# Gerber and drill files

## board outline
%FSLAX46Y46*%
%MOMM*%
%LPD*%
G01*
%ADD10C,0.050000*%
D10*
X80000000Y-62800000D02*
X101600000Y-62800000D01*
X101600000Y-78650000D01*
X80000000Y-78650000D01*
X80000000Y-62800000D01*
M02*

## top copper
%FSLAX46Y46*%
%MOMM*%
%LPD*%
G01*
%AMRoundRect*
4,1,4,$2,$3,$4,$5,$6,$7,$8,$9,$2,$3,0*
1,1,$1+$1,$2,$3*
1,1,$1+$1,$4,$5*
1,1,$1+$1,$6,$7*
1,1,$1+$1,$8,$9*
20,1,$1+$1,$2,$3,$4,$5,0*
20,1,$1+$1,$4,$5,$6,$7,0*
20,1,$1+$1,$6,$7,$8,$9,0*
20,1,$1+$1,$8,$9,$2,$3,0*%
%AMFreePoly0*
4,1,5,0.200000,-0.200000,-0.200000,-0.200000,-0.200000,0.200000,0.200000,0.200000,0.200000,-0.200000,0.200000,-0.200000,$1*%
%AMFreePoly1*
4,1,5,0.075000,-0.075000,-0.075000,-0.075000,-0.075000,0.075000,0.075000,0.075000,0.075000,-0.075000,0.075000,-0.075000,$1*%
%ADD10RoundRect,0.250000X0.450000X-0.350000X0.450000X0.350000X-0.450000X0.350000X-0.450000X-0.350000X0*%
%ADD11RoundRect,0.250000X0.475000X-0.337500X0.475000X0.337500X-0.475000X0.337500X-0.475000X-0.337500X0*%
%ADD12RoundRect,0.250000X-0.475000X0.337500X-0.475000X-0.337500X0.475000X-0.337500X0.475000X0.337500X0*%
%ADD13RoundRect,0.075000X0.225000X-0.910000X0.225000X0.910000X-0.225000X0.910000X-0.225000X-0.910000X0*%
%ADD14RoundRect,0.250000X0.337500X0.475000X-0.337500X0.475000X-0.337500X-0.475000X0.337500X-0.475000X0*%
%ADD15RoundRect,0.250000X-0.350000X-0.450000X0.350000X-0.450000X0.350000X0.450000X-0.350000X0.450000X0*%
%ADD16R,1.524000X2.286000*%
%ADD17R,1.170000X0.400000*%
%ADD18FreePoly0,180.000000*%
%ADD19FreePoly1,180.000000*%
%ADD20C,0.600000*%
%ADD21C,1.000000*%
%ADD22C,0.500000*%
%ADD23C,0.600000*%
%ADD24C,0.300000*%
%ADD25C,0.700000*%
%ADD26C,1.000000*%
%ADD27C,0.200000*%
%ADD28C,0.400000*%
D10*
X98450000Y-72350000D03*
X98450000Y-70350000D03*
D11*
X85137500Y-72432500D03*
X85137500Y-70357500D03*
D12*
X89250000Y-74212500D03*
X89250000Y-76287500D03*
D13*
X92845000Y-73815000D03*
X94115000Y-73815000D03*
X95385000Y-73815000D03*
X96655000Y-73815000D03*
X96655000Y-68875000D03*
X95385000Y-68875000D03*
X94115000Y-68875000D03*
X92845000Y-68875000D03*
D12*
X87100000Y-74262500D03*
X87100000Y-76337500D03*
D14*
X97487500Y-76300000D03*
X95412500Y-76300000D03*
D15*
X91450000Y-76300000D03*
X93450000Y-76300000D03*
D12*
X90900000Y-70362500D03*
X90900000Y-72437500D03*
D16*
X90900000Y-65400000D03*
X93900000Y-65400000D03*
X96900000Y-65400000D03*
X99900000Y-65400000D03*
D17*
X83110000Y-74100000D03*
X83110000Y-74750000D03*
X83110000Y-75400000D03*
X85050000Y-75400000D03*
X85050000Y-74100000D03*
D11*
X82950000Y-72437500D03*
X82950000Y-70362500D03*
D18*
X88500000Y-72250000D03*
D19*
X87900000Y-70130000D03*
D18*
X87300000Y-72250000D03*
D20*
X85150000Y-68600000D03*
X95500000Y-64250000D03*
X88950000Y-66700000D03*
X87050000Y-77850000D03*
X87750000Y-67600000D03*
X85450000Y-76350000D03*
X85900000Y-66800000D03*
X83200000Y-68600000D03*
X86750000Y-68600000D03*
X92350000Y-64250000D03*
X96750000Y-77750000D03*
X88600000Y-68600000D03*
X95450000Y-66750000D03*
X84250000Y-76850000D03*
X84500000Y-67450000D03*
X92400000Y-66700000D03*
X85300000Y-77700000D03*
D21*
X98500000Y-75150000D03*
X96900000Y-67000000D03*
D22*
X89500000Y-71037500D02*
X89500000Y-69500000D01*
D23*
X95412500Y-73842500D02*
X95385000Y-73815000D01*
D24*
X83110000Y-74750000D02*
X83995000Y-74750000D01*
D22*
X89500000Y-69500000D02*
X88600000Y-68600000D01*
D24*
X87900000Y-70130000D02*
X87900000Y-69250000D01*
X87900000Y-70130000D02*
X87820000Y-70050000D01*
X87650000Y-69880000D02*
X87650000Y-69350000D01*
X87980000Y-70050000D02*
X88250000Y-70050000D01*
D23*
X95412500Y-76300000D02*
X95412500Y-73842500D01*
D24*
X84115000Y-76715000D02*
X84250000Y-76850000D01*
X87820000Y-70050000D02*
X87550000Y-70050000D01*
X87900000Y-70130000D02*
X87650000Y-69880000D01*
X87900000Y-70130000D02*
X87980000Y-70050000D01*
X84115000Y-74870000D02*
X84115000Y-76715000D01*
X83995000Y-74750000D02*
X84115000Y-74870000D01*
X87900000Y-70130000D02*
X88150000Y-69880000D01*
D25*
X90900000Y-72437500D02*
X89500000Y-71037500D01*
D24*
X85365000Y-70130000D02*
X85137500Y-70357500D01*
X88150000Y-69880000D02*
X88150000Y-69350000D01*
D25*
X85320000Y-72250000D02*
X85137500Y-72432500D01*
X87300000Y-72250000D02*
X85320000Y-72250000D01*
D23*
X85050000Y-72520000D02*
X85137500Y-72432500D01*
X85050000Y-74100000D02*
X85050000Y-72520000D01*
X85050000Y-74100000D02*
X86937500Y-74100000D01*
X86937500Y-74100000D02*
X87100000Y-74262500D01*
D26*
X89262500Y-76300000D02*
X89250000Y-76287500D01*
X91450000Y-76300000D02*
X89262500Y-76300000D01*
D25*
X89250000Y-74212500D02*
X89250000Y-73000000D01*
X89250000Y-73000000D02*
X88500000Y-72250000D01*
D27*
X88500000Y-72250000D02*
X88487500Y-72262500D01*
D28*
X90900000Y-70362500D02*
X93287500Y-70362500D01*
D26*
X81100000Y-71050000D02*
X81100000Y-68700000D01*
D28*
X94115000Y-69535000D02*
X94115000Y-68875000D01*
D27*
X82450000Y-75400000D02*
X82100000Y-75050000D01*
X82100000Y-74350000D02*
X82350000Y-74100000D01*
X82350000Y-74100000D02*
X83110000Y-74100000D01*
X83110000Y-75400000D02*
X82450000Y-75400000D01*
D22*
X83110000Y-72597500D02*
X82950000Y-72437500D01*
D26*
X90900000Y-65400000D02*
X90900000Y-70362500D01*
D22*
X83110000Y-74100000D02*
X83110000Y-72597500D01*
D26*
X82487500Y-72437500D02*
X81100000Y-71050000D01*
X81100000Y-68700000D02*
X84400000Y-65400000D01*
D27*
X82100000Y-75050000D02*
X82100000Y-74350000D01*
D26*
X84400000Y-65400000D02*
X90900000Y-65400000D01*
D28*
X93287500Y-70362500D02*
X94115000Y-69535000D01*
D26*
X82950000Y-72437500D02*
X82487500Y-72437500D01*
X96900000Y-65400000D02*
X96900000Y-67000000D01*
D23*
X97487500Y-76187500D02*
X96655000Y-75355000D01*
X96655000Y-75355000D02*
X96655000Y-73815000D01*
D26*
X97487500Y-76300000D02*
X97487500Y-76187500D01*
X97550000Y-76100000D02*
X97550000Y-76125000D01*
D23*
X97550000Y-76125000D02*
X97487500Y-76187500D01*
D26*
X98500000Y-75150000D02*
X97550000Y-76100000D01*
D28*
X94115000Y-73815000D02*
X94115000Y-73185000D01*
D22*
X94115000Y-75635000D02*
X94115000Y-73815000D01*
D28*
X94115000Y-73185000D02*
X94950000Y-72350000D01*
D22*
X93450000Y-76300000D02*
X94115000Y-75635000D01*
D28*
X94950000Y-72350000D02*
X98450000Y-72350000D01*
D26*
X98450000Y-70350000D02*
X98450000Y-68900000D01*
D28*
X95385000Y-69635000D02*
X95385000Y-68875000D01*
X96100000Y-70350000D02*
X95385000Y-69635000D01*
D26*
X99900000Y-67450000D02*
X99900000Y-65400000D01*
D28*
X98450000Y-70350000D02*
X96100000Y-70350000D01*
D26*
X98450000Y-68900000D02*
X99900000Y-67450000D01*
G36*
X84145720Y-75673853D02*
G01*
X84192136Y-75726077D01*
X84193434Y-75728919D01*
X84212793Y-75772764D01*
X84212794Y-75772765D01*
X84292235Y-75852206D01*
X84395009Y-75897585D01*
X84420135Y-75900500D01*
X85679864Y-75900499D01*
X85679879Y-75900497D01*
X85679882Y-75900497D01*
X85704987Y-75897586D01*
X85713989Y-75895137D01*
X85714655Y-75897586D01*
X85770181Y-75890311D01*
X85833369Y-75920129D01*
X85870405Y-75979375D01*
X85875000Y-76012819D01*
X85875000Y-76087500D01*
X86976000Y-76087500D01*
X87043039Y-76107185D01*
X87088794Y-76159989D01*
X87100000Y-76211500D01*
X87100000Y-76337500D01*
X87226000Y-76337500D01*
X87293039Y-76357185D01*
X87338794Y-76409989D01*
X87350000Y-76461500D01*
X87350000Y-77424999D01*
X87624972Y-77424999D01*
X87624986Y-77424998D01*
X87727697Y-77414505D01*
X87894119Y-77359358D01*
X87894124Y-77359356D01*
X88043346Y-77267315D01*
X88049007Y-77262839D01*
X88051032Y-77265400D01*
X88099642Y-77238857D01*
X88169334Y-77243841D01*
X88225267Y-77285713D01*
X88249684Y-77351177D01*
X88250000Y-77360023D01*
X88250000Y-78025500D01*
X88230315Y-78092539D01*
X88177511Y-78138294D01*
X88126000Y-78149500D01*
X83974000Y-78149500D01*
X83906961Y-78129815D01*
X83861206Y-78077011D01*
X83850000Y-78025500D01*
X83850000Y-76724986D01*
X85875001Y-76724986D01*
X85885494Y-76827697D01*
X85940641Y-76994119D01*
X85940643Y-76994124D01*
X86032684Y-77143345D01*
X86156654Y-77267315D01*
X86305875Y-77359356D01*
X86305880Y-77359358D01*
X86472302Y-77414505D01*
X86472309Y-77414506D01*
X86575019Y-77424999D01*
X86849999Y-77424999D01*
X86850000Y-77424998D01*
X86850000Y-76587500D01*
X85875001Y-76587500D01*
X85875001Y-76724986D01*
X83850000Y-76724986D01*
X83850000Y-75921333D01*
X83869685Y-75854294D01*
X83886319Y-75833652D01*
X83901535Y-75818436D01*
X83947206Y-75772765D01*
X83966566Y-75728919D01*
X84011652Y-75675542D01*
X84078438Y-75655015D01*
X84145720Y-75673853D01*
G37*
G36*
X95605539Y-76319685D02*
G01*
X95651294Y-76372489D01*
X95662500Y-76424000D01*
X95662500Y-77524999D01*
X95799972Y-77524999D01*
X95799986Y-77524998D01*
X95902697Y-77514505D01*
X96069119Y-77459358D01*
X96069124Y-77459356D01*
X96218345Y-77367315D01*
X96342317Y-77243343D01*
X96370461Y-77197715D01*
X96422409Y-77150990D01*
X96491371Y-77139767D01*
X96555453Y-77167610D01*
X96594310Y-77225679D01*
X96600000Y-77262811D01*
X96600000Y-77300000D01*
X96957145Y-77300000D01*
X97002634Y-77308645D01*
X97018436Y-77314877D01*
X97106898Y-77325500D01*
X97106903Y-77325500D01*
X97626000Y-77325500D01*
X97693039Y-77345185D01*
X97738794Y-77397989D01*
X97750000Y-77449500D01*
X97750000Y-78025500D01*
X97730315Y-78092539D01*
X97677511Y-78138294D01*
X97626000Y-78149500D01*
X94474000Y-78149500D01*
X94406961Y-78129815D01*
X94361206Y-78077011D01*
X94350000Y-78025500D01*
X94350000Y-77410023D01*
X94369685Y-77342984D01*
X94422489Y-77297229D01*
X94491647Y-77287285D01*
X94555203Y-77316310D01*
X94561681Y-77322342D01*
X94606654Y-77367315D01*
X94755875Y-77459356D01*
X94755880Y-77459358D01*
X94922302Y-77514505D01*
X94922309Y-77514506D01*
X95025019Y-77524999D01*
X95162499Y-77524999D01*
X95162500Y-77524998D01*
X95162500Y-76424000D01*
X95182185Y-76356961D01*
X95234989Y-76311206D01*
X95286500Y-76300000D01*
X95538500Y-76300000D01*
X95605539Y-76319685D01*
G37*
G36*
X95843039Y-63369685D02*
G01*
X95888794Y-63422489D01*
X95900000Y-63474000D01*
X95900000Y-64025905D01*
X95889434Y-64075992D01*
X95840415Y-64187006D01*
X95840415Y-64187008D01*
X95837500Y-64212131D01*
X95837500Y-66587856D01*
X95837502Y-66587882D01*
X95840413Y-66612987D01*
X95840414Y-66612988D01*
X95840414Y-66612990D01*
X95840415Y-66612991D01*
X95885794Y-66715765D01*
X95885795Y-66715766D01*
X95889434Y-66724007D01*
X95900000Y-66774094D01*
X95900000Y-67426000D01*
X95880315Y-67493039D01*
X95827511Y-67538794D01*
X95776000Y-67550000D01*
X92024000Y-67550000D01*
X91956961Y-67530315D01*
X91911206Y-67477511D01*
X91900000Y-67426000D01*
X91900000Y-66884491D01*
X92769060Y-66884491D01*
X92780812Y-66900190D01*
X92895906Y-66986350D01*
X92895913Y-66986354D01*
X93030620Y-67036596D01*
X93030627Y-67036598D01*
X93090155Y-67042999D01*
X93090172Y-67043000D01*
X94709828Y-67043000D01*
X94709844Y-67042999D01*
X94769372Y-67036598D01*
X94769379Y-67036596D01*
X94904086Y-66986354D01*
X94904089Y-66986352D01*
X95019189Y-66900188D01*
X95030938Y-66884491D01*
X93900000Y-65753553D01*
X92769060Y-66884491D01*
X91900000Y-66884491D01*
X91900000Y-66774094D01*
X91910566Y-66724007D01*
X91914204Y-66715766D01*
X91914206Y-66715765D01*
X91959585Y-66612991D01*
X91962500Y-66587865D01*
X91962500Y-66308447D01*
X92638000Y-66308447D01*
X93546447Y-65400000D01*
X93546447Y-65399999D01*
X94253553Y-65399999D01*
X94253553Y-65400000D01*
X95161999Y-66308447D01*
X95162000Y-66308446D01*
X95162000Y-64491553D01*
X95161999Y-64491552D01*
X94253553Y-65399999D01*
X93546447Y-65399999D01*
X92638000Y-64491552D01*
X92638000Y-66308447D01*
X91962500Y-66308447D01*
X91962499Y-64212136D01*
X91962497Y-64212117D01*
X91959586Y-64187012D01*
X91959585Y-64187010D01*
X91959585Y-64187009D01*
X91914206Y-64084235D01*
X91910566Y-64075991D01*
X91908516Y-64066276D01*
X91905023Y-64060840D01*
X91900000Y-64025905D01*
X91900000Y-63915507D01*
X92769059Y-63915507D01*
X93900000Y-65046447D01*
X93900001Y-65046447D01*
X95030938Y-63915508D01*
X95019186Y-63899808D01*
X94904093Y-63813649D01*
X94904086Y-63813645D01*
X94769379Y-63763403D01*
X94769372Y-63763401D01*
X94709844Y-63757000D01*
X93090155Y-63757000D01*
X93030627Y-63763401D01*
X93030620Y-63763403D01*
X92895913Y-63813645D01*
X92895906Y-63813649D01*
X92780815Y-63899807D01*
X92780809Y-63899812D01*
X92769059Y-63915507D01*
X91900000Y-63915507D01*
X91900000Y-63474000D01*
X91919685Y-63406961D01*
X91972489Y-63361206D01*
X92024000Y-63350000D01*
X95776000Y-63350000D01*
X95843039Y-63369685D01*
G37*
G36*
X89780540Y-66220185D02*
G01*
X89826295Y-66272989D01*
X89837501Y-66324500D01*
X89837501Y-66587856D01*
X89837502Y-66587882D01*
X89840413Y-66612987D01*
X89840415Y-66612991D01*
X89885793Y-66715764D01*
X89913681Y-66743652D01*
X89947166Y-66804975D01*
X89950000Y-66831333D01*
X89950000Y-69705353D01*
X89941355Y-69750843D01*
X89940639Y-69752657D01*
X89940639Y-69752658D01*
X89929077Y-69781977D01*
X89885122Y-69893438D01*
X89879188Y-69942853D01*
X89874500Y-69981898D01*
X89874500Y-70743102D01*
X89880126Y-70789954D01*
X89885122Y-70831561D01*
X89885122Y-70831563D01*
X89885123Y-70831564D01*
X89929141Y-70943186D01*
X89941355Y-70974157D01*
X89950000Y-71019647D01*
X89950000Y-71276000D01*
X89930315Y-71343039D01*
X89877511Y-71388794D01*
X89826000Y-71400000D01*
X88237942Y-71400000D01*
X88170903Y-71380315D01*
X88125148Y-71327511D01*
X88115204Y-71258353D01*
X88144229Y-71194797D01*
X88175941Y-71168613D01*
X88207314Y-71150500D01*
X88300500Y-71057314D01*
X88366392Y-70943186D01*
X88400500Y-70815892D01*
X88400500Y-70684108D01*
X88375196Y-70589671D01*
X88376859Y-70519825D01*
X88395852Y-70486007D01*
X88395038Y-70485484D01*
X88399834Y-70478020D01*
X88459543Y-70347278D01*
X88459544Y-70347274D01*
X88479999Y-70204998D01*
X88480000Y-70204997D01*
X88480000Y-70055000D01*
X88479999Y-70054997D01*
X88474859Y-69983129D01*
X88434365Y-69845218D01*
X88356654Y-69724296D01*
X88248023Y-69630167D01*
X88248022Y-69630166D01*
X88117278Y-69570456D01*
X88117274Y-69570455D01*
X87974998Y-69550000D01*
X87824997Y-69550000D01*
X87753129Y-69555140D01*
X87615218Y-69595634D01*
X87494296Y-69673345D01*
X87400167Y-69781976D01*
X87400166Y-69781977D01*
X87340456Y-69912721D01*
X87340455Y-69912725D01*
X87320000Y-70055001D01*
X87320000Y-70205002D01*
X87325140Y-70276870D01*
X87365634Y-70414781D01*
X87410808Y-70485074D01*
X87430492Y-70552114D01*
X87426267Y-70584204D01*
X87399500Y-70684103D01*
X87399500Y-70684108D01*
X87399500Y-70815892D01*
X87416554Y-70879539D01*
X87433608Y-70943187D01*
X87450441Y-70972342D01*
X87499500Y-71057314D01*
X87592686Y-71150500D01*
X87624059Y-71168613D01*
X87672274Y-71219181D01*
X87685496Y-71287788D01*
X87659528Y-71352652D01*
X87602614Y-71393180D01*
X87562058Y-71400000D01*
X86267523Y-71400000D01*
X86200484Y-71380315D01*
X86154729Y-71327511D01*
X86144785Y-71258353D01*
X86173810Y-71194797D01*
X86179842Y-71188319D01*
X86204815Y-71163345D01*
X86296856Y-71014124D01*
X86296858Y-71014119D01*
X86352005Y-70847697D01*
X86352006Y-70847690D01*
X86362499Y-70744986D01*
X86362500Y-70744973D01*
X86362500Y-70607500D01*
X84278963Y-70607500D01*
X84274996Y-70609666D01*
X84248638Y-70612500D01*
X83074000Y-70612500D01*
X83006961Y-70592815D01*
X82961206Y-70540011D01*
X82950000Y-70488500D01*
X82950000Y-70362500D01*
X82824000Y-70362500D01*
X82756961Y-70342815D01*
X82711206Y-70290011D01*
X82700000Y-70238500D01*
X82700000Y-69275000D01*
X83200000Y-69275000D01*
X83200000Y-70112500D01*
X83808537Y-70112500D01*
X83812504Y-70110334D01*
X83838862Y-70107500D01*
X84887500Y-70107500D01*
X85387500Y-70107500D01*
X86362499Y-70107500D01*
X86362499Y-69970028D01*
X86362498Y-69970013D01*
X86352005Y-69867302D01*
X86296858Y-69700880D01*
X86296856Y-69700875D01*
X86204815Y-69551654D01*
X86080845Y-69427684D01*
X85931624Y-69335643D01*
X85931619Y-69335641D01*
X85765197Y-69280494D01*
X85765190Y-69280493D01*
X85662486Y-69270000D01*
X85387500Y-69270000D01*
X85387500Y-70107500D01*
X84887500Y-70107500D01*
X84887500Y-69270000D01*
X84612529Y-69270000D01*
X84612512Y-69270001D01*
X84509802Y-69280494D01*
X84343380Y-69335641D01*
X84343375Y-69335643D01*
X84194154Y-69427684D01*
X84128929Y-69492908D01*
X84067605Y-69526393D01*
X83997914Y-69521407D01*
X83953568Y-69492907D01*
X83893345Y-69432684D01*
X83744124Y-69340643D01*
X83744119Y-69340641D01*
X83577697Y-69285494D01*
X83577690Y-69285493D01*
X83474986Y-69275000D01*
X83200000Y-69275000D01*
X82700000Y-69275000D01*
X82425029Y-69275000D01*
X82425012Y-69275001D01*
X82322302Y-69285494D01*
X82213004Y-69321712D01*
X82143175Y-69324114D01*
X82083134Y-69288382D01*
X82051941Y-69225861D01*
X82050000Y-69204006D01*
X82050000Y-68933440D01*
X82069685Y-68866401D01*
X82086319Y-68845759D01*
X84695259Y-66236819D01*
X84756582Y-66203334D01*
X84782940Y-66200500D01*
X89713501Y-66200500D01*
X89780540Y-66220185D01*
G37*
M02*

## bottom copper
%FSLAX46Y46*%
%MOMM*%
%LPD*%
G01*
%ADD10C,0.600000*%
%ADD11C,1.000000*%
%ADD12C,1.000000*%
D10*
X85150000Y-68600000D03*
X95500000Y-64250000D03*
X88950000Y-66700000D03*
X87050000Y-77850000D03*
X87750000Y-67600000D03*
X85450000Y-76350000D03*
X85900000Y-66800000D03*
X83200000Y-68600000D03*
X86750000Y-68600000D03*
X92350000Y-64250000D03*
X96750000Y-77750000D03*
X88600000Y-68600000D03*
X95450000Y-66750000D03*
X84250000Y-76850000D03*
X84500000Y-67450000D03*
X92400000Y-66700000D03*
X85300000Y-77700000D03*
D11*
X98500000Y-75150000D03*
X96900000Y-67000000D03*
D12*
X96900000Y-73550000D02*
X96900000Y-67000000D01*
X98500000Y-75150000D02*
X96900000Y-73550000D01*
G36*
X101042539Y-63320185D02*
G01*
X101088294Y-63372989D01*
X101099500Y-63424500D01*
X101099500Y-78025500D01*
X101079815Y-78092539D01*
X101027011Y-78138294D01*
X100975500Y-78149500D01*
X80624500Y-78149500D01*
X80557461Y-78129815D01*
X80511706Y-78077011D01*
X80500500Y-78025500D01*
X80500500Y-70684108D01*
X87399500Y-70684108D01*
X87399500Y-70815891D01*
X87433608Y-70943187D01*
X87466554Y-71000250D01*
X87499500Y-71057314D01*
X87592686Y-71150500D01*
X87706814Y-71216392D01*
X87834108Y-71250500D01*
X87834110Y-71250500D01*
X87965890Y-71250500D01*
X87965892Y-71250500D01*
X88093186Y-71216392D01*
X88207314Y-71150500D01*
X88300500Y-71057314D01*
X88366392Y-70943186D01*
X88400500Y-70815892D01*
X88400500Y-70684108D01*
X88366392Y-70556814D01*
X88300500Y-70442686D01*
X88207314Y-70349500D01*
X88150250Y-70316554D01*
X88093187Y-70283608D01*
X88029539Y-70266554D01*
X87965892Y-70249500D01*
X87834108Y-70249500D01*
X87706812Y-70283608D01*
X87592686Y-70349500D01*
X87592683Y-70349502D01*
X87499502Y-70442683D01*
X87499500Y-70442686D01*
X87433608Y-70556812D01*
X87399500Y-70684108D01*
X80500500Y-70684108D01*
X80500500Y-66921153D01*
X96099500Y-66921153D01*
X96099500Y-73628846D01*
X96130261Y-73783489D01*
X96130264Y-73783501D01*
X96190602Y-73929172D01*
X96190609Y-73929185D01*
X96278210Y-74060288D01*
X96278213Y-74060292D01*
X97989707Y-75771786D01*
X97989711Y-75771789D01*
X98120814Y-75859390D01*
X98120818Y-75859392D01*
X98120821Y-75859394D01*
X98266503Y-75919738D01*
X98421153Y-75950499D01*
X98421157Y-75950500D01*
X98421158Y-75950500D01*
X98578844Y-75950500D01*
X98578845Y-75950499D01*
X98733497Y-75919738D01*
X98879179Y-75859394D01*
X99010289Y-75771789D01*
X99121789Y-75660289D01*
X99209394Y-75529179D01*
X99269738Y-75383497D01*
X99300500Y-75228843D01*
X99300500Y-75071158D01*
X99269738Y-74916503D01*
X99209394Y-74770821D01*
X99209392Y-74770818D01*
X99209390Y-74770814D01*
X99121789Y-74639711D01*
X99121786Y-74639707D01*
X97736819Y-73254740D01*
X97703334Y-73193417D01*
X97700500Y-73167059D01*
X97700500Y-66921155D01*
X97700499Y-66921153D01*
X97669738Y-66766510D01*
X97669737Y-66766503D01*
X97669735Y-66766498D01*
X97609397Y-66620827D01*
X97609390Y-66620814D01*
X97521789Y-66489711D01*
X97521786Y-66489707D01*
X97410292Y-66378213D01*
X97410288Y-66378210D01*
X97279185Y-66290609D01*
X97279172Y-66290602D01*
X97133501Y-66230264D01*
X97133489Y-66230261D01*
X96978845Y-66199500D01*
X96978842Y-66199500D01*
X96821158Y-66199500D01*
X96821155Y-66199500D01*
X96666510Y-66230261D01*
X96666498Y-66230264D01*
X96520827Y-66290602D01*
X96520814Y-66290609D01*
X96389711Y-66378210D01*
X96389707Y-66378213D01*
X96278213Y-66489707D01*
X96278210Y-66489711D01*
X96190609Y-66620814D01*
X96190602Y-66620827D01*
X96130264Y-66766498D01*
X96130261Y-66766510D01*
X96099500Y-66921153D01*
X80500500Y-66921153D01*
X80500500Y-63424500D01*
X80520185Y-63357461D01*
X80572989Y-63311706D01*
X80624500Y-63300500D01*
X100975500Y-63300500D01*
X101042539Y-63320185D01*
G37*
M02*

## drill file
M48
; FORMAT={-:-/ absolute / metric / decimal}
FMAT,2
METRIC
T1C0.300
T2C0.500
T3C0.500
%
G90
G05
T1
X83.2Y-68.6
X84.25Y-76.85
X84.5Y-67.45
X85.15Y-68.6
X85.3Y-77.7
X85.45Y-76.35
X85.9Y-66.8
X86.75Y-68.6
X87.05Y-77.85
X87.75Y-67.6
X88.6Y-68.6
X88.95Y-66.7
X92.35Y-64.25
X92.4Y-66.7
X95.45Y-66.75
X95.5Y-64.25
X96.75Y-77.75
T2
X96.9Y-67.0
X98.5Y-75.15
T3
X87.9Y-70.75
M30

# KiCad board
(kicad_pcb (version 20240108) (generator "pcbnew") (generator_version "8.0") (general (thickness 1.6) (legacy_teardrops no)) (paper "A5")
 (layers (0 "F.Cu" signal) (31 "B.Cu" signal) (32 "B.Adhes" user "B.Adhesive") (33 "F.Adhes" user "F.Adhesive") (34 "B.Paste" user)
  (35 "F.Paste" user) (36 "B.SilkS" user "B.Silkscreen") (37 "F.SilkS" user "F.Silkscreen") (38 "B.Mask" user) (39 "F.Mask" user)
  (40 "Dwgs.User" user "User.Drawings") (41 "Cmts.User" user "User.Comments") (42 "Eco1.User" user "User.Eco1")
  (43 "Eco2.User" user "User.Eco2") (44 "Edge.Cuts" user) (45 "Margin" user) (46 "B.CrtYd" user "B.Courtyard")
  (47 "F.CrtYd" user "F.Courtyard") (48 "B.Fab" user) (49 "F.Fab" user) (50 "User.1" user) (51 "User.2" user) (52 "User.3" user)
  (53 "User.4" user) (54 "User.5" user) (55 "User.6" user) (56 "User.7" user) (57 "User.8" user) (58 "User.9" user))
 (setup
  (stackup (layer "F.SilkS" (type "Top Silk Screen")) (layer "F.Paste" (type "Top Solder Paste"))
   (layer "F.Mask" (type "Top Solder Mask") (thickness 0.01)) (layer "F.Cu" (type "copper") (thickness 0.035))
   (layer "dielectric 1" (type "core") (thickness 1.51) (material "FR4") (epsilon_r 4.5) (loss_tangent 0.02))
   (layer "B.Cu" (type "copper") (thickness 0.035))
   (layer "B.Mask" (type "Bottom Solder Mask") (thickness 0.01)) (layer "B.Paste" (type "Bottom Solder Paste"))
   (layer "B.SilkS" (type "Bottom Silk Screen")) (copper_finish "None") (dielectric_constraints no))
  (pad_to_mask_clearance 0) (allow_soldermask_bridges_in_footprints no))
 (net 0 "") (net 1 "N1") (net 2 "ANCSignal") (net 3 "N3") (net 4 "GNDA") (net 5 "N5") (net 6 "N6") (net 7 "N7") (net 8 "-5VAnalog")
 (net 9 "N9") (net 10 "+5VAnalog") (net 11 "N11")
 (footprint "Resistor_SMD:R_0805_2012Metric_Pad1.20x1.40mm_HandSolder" (layer "F.Cu") (at 98.45 71.35 90)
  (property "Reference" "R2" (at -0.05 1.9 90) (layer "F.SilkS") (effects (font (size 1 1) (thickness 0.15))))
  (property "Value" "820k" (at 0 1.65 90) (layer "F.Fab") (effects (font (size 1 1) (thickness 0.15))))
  (pad "1" smd roundrect (at -1 0 90) (size 1.2 1.4) (layers "F.Cu" "F.Paste" "F.Mask") (roundrect_rratio 0.208333) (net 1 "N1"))
  (pad "2" smd roundrect (at 1 0 90) (size 1.2 1.4) (layers "F.Cu" "F.Paste" "F.Mask") (roundrect_rratio 0.208333) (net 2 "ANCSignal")))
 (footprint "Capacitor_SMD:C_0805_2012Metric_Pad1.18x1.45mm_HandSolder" (layer "F.Cu") (at 85.1375 71.395 90)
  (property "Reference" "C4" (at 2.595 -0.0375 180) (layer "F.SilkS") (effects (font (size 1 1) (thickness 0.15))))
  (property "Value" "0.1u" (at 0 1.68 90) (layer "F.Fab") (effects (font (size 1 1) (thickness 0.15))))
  (pad "1" smd roundrect (at -1.0375 0 90) (size 1.175 1.45) (layers "F.Cu" "F.Paste" "F.Mask") (roundrect_rratio 0.212766) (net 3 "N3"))
  (pad "2" smd roundrect (at 1.0375 0 90) (size 1.175 1.45) (layers "F.Cu" "F.Paste" "F.Mask") (roundrect_rratio 0.212766) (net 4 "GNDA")))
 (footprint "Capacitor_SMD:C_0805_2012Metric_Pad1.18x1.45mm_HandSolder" (layer "F.Cu") (at 89.25 75.25 -90)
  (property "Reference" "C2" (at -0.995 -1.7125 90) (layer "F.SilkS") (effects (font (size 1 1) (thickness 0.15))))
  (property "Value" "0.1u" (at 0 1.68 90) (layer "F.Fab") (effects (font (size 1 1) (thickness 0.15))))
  (pad "1" smd roundrect (at -1.0375 0 270) (size 1.175 1.45) (layers "F.Cu" "F.Paste" "F.Mask") (roundrect_rratio 0.212766) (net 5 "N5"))
  (pad "2" smd roundrect (at 1.0375 0 270) (size 1.175 1.45) (layers "F.Cu" "F.Paste" "F.Mask") (roundrect_rratio 0.212766) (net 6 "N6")))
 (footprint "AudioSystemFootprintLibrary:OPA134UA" (layer "F.Cu") (at 94.75 71.345 90)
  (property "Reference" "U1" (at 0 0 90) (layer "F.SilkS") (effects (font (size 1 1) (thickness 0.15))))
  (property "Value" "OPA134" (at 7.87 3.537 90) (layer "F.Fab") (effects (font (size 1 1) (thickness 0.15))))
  (pad "1" smd roundrect (at -2.47 -1.905 90) (size 1.97 0.6) (layers "F.Cu" "F.Paste" "F.Mask") (roundrect_rratio 0.125) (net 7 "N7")
   (solder_mask_margin 0.102))
  (pad "2" smd roundrect (at -2.47 -0.635 90) (size 1.97 0.6) (layers "F.Cu" "F.Paste" "F.Mask") (roundrect_rratio 0.125) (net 1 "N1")
   (solder_mask_margin 0.102))
  (pad "3" smd roundrect (at -2.47 0.635 90) (size 1.97 0.6) (layers "F.Cu" "F.Paste" "F.Mask") (roundrect_rratio 0.125) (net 4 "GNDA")
   (solder_mask_margin 0.102))
  (pad "4" smd roundrect (at -2.47 1.905 90) (size 1.97 0.6) (layers "F.Cu" "F.Paste" "F.Mask") (roundrect_rratio 0.125) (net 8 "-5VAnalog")
   (solder_mask_margin 0.102))
  (pad "5" smd roundrect (at 2.47 1.905 90) (size 1.97 0.6) (layers "F.Cu" "F.Paste" "F.Mask") (roundrect_rratio 0.125) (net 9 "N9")
   (solder_mask_margin 0.102))
  (pad "6" smd roundrect (at 2.47 0.635 90) (size 1.97 0.6) (layers "F.Cu" "F.Paste" "F.Mask") (roundrect_rratio 0.125) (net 2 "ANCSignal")
   (solder_mask_margin 0.102))
  (pad "7" smd roundrect (at 2.47 -0.635 90) (size 1.97 0.6) (layers "F.Cu" "F.Paste" "F.Mask") (roundrect_rratio 0.125)
   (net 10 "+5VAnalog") (solder_mask_margin 0.102))
  (pad "8" smd roundrect (at 2.47 -1.905 90) (size 1.97 0.6) (layers "F.Cu" "F.Paste" "F.Mask") (roundrect_rratio 0.125) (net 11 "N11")
   (solder_mask_margin 0.102)))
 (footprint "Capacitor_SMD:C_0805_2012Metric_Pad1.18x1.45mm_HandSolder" (layer "F.Cu") (at 87.1 75.3 -90)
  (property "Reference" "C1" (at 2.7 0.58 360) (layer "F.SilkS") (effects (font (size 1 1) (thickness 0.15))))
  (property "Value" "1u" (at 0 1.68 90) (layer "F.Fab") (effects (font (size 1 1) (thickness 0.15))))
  (pad "1" smd roundrect (at -1.0375 0 270) (size 1.175 1.45) (layers "F.Cu" "F.Paste" "F.Mask") (roundrect_rratio 0.212766) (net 3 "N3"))
  (pad "2" smd roundrect (at 1.0375 0 270) (size 1.175 1.45) (layers "F.Cu" "F.Paste" "F.Mask") (roundrect_rratio 0.212766) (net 4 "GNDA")))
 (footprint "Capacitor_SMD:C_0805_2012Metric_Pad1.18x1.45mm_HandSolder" (layer "F.Cu") (at 96.45 76.3 180)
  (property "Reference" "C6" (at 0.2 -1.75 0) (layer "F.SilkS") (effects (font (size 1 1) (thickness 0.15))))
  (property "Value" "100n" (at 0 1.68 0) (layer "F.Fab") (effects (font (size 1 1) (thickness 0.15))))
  (pad "1" smd roundrect (at -1.0375 0 180) (size 1.175 1.45) (layers "F.Cu" "F.Paste" "F.Mask") (roundrect_rratio 0.212766)
   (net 8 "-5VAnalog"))
  (pad "2" smd roundrect (at 1.0375 0 180) (size 1.175 1.45) (layers "F.Cu" "F.Paste" "F.Mask") (roundrect_rratio 0.212766) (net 4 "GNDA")))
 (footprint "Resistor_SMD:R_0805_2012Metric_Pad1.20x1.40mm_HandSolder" (layer "F.Cu") (at 92.45 76.3)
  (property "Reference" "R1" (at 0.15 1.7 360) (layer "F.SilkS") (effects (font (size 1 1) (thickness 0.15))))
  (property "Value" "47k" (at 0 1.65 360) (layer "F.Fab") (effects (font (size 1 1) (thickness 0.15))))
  (pad "1" smd roundrect (at -1 0) (size 1.2 1.4) (layers "F.Cu" "F.Paste" "F.Mask") (roundrect_rratio 0.208333) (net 6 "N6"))
  (pad "2" smd roundrect (at 1 0) (size 1.2 1.4) (layers "F.Cu" "F.Paste" "F.Mask") (roundrect_rratio 0.208333) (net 1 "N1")))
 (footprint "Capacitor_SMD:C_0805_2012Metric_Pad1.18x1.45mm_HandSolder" (layer "F.Cu") (at 90.9 71.4 -90)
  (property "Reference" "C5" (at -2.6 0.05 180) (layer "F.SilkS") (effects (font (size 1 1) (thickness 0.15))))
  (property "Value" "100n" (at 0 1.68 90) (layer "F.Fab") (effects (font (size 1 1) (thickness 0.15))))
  (pad "1" smd roundrect (at -1.0375 0 270) (size 1.175 1.45) (layers "F.Cu" "F.Paste" "F.Mask") (roundrect_rratio 0.212766)
   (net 10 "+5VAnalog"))
  (pad "2" smd roundrect (at 1.0375 0 270) (size 1.175 1.45) (layers "F.Cu" "F.Paste" "F.Mask") (roundrect_rratio 0.212766) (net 4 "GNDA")))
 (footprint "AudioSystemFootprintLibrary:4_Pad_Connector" (layer "F.Cu") (at 94.9 63.4)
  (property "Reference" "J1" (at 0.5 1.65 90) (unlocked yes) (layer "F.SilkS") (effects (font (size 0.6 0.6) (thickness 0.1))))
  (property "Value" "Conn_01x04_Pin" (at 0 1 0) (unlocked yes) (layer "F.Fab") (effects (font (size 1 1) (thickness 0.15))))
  (pad "1" smd rect (at -4 2 90) (size 2.286 1.524) (layers "F.Cu" "F.Paste" "F.Mask") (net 10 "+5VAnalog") (thermal_bridge_angle 45))
  (pad "2" smd rect (at -1 2 90) (size 2.286 1.524) (layers "F.Cu" "F.Paste" "F.Mask") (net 4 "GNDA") (thermal_bridge_angle 45))
  (pad "3" smd rect (at 2 2 90) (size 2.286 1.524) (layers "F.Cu" "F.Paste" "F.Mask") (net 8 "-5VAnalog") (thermal_bridge_angle 45))
  (pad "4" smd rect (at 5 2 90) (size 2.286 1.524) (layers "F.Cu" "F.Paste" "F.Mask") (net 2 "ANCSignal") (thermal_bridge_angle 45)))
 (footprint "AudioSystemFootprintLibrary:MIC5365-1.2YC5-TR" (layer "F.Cu") (at 84.08 74.75)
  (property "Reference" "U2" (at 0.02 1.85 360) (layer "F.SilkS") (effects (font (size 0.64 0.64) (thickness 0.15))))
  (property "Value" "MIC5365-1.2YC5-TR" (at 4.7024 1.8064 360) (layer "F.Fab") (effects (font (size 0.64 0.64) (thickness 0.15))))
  (pad "1" smd rect (at -0.97 -0.65) (size 1.17 0.4) (layers "F.Cu" "F.Paste" "F.Mask") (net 10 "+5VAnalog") (solder_mask_margin 0.102))
  (pad "2" smd rect (at -0.97 0) (size 1.17 0.4) (layers "F.Cu" "F.Paste" "F.Mask") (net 4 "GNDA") (solder_mask_margin 0.102))
  (pad "3" smd rect (at -0.97 0.65) (size 1.17 0.4) (layers "F.Cu" "F.Paste" "F.Mask") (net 10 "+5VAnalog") (solder_mask_margin 0.102))
  (pad "4" smd rect (at 0.97 0.65) (size 1.17 0.4) (layers "F.Cu" "F.Paste" "F.Mask") (solder_mask_margin 0.102))
  (pad "5" smd rect (at 0.97 -0.65) (size 1.17 0.4) (layers "F.Cu" "F.Paste" "F.Mask") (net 3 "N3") (solder_mask_margin 0.102)))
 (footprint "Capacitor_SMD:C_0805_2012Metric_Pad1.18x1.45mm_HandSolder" (layer "F.Cu") (at 82.95 71.4 90)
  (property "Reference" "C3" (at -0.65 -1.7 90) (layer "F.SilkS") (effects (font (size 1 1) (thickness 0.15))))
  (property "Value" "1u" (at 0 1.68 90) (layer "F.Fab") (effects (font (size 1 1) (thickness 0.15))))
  (pad "1" smd roundrect (at -1.0375 0 90) (size 1.175 1.45) (layers "F.Cu" "F.Paste" "F.Mask") (roundrect_rratio 0.212766)
   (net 10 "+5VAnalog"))
  (pad "2" smd roundrect (at 1.0375 0 90) (size 1.175 1.45) (layers "F.Cu" "F.Paste" "F.Mask") (roundrect_rratio 0.212766) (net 4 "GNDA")))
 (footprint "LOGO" (layer "F.Cu") (at 85.6 64)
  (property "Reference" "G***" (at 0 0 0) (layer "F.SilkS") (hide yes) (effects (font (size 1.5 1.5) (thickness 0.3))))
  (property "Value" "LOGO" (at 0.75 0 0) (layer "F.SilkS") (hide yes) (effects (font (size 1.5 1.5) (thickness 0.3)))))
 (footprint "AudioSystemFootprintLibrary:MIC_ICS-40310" (layer "F.Cu") (at 87.9 70.75 180)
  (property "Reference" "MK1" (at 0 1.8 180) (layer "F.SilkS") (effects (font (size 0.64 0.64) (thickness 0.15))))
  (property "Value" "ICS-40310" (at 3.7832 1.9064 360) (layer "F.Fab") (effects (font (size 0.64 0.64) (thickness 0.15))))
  (pad "" np_thru_hole circle (at 0 0 180) (size 0.5 0.5) (drill 0.5) (layers "*.Cu" "*.Mask"))
  (pad "1" smd custom (at -0.6 -1.5 180) (size 0.4 0.4) (layers "F.Cu") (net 5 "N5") (options (clearance outline) (anchor rect))
   (primitives))
  (pad "2" smd custom (at 0 0.62 180) (size 0.15 0.15) (layers "F.Cu") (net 4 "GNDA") (options (clearance outline) (anchor rect))
   (primitives))
  (pad "3" smd custom (at 0.6 -1.5 180) (size 0.4 0.4) (layers "F.Cu") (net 3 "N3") (options (clearance outline) (anchor rect)) (primitives)))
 (gr_rect (start 80 62.8) (end 101.6 78.65) (stroke (width 0.05) (type default)) (fill none) (layer "Edge.Cuts"))
 (segment (start 89.5 71.0375) (end 89.5 69.5) (width 0.5) (layer "F.Cu") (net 4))
 (segment (start 95.4125 73.8425) (end 95.385 73.815) (width 0.6) (layer "F.Cu") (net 4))
 (segment (start 83.11 74.75) (end 83.995 74.75) (width 0.3) (layer "F.Cu") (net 4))
 (segment (start 89.5 69.5) (end 88.6 68.6) (width 0.5) (layer "F.Cu") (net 4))
 (segment (start 87.9 70.13) (end 87.9 69.25) (width 0.3) (layer "F.Cu") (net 4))
 (segment (start 87.9 70.13) (end 87.82 70.05) (width 0.3) (layer "F.Cu") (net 4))
 (segment (start 87.65 69.88) (end 87.65 69.35) (width 0.3) (layer "F.Cu") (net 4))
 (segment (start 87.98 70.05) (end 88.25 70.05) (width 0.3) (layer "F.Cu") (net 4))
 (segment (start 95.4125 76.3) (end 95.4125 73.8425) (width 0.6) (layer "F.Cu") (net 4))
 (segment (start 84.115 76.715) (end 84.25 76.85) (width 0.3) (layer "F.Cu") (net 4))
 (segment (start 87.82 70.05) (end 87.55 70.05) (width 0.3) (layer "F.Cu") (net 4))
 (segment (start 87.9 70.13) (end 87.65 69.88) (width 0.3) (layer "F.Cu") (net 4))
 (segment (start 87.9 70.13) (end 87.98 70.05) (width 0.3) (layer "F.Cu") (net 4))
 (segment (start 84.115 74.87) (end 84.115 76.715) (width 0.3) (layer "F.Cu") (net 4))
 (segment (start 83.995 74.75) (end 84.115 74.87) (width 0.3) (layer "F.Cu") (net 4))
 (segment (start 87.9 70.13) (end 88.15 69.88) (width 0.3) (layer "F.Cu") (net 4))
 (segment (start 90.9 72.4375) (end 89.5 71.0375) (width 0.7) (layer "F.Cu") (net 4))
 (segment (start 85.365 70.13) (end 85.1375 70.3575) (width 0.3) (layer "F.Cu") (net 4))
 (segment (start 88.15 69.88) (end 88.15 69.35) (width 0.3) (layer "F.Cu") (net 4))
 (via (at 85.15 68.6) (size 0.6) (drill 0.3) (layers "F.Cu" "B.Cu") (free yes) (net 4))
 (via (at 95.5 64.25) (size 0.6) (drill 0.3) (layers "F.Cu" "B.Cu") (free yes) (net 4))
 (via (at 88.95 66.7) (size 0.6) (drill 0.3) (layers "F.Cu" "B.Cu") (free yes) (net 4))
 (via (at 87.05 77.85) (size 0.6) (drill 0.3) (layers "F.Cu" "B.Cu") (free yes) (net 4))
 (via (at 87.75 67.6) (size 0.6) (drill 0.3) (layers "F.Cu" "B.Cu") (free yes) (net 4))
 (via (at 85.45 76.35) (size 0.6) (drill 0.3) (layers "F.Cu" "B.Cu") (free yes) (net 4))
 (via (at 85.9 66.8) (size 0.6) (drill 0.3) (layers "F.Cu" "B.Cu") (free yes) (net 4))
 (via (at 83.2 68.6) (size 0.6) (drill 0.3) (layers "F.Cu" "B.Cu") (free yes) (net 4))
 (via (at 86.75 68.6) (size 0.6) (drill 0.3) (layers "F.Cu" "B.Cu") (free yes) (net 4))
 (via (at 92.35 64.25) (size 0.6) (drill 0.3) (layers "F.Cu" "B.Cu") (free yes) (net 4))
 (via (at 96.75 77.75) (size 0.6) (drill 0.3) (layers "F.Cu" "B.Cu") (free yes) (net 4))
 (via (at 88.6 68.6) (size 0.6) (drill 0.3) (layers "F.Cu" "B.Cu") (free yes) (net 4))
 (via (at 95.45 66.75) (size 0.6) (drill 0.3) (layers "F.Cu" "B.Cu") (free yes) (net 4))
 (via (at 84.25 76.85) (size 0.6) (drill 0.3) (layers "F.Cu" "B.Cu") (free yes) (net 4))
 (via (at 84.5 67.45) (size 0.6) (drill 0.3) (layers "F.Cu" "B.Cu") (free yes) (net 4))
 (via (at 92.4 66.7) (size 0.6) (drill 0.3) (layers "F.Cu" "B.Cu") (free yes) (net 4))
 (via (at 85.3 77.7) (size 0.6) (drill 0.3) (layers "F.Cu" "B.Cu") (free yes) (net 4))
 (segment (start 85.32 72.25) (end 85.1375 72.4325) (width 0.7) (layer "F.Cu") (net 3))
 (segment (start 87.3 72.25) (end 85.32 72.25) (width 0.7) (layer "F.Cu") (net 3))
 (segment (start 85.05 72.52) (end 85.1375 72.4325) (width 0.6) (layer "F.Cu") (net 3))
 (segment (start 85.05 74.1) (end 85.05 72.52) (width 0.6) (layer "F.Cu") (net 3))
 (segment (start 85.05 74.1) (end 86.9375 74.1) (width 0.6) (layer "F.Cu") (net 3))
 (segment (start 86.9375 74.1) (end 87.1 74.2625) (width 0.6) (layer "F.Cu") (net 3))
 (segment (start 89.2625 76.3) (end 89.25 76.2875) (width 1) (layer "F.Cu") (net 6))
 (segment (start 91.45 76.3) (end 89.2625 76.3) (width 1) (layer "F.Cu") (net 6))
 (segment (start 89.25 74.2125) (end 89.25 73) (width 0.7) (layer "F.Cu") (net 5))
 (segment (start 89.25 73) (end 88.5 72.25) (width 0.7) (layer "F.Cu") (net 5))
 (segment (start 88.5 72.25) (end 88.4875 72.2625) (width 0.2) (layer "F.Cu") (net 5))
 (segment (start 90.9 70.3625) (end 93.2875 70.3625) (width 0.4) (layer "F.Cu") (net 10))
 (segment (start 81.1 71.05) (end 81.1 68.7) (width 1) (layer "F.Cu") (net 10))
 (segment (start 94.115 69.535) (end 94.115 68.875) (width 0.4) (layer "F.Cu") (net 10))
 (segment (start 82.45 75.4) (end 82.1 75.05) (width 0.2) (layer "F.Cu") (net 10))
 (segment (start 82.1 74.35) (end 82.35 74.1) (width 0.2) (layer "F.Cu") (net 10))
 (segment (start 82.35 74.1) (end 83.11 74.1) (width 0.2) (layer "F.Cu") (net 10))
 (segment (start 83.11 75.4) (end 82.45 75.4) (width 0.2) (layer "F.Cu") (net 10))
 (segment (start 83.11 72.5975) (end 82.95 72.4375) (width 0.5) (layer "F.Cu") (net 10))
 (segment (start 90.9 65.4) (end 90.9 70.3625) (width 1) (layer "F.Cu") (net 10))
 (segment (start 83.11 74.1) (end 83.11 72.5975) (width 0.5) (layer "F.Cu") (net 10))
 (segment (start 82.4875 72.4375) (end 81.1 71.05) (width 1) (layer "F.Cu") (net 10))
 (segment (start 81.1 68.7) (end 84.4 65.4) (width 1) (layer "F.Cu") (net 10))
 (segment (start 82.1 75.05) (end 82.1 74.35) (width 0.2) (layer "F.Cu") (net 10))
 (segment (start 84.4 65.4) (end 90.9 65.4) (width 1) (layer "F.Cu") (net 10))
 (segment (start 93.2875 70.3625) (end 94.115 69.535) (width 0.4) (layer "F.Cu") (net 10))
 (segment (start 82.95 72.4375) (end 82.4875 72.4375) (width 1) (layer "F.Cu") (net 10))
 (segment (start 96.9 65.4) (end 96.9 67) (width 1) (layer "F.Cu") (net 8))
 (segment (start 97.4875 76.1875) (end 96.655 75.355) (width 0.6) (layer "F.Cu") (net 8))
 (segment (start 96.655 75.355) (end 96.655 73.815) (width 0.6) (layer "F.Cu") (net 8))
 (segment (start 97.4875 76.3) (end 97.4875 76.1875) (width 1) (layer "F.Cu") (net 8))
 (segment (start 97.55 76.1) (end 97.55 76.125) (width 1) (layer "F.Cu") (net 8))
 (segment (start 97.55 76.125) (end 97.4875 76.1875) (width 0.6) (layer "F.Cu") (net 8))
 (segment (start 98.5 75.15) (end 97.55 76.1) (width 1) (layer "F.Cu") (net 8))
 (via (at 98.5 75.15) (size 1) (drill 0.5) (layers "F.Cu" "B.Cu") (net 8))
 (via (at 96.9 67) (size 1) (drill 0.5) (layers "F.Cu" "B.Cu") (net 8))
 (segment (start 96.9 73.55) (end 96.9 67) (width 1) (layer "B.Cu") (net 8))
 (segment (start 98.5 75.15) (end 96.9 73.55) (width 1) (layer "B.Cu") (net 8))
 (segment (start 94.115 73.815) (end 94.115 73.185) (width 0.4) (layer "F.Cu") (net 1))
 (segment (start 94.115 75.635) (end 94.115 73.815) (width 0.5) (layer "F.Cu") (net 1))
 (segment (start 94.115 73.185) (end 94.95 72.35) (width 0.4) (layer "F.Cu") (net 1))
 (segment (start 93.45 76.3) (end 94.115 75.635) (width 0.5) (layer "F.Cu") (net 1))
 (segment (start 94.95 72.35) (end 98.45 72.35) (width 0.4) (layer "F.Cu") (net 1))
 (segment (start 98.45 70.35) (end 98.45 68.9) (width 1) (layer "F.Cu") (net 2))
 (segment (start 95.385 69.635) (end 95.385 68.875) (width 0.4) (layer "F.Cu") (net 2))
 (segment (start 96.1 70.35) (end 95.385 69.635) (width 0.4) (layer "F.Cu") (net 2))
 (segment (start 99.9 67.45) (end 99.9 65.4) (width 1) (layer "F.Cu") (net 2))
 (segment (start 98.45 70.35) (end 96.1 70.35) (width 0.4) (layer "F.Cu") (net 2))
 (segment (start 98.45 68.9) (end 99.9 67.45) (width 1) (layer "F.Cu") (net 2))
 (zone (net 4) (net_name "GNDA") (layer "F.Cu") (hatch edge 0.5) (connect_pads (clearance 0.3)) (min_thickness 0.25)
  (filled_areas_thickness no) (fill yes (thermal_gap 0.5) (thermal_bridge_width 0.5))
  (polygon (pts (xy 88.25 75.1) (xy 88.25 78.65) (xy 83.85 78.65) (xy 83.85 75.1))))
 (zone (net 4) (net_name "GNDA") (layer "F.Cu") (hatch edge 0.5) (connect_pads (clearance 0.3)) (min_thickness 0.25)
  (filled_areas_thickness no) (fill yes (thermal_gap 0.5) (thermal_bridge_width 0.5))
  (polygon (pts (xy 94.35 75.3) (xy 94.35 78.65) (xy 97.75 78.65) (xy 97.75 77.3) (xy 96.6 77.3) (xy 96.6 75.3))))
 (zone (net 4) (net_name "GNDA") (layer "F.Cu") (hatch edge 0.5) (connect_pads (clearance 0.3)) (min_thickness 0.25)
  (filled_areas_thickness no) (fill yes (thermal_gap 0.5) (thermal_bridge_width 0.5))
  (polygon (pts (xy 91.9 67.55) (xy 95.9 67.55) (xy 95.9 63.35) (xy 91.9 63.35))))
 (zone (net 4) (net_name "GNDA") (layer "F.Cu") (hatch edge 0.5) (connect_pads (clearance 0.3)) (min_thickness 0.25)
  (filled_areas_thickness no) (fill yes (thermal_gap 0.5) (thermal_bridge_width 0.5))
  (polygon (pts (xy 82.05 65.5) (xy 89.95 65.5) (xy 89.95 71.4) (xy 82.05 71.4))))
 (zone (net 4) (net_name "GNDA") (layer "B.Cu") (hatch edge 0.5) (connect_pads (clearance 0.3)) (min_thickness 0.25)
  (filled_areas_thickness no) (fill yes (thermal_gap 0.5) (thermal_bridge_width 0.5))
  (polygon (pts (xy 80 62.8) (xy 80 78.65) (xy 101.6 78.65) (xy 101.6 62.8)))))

